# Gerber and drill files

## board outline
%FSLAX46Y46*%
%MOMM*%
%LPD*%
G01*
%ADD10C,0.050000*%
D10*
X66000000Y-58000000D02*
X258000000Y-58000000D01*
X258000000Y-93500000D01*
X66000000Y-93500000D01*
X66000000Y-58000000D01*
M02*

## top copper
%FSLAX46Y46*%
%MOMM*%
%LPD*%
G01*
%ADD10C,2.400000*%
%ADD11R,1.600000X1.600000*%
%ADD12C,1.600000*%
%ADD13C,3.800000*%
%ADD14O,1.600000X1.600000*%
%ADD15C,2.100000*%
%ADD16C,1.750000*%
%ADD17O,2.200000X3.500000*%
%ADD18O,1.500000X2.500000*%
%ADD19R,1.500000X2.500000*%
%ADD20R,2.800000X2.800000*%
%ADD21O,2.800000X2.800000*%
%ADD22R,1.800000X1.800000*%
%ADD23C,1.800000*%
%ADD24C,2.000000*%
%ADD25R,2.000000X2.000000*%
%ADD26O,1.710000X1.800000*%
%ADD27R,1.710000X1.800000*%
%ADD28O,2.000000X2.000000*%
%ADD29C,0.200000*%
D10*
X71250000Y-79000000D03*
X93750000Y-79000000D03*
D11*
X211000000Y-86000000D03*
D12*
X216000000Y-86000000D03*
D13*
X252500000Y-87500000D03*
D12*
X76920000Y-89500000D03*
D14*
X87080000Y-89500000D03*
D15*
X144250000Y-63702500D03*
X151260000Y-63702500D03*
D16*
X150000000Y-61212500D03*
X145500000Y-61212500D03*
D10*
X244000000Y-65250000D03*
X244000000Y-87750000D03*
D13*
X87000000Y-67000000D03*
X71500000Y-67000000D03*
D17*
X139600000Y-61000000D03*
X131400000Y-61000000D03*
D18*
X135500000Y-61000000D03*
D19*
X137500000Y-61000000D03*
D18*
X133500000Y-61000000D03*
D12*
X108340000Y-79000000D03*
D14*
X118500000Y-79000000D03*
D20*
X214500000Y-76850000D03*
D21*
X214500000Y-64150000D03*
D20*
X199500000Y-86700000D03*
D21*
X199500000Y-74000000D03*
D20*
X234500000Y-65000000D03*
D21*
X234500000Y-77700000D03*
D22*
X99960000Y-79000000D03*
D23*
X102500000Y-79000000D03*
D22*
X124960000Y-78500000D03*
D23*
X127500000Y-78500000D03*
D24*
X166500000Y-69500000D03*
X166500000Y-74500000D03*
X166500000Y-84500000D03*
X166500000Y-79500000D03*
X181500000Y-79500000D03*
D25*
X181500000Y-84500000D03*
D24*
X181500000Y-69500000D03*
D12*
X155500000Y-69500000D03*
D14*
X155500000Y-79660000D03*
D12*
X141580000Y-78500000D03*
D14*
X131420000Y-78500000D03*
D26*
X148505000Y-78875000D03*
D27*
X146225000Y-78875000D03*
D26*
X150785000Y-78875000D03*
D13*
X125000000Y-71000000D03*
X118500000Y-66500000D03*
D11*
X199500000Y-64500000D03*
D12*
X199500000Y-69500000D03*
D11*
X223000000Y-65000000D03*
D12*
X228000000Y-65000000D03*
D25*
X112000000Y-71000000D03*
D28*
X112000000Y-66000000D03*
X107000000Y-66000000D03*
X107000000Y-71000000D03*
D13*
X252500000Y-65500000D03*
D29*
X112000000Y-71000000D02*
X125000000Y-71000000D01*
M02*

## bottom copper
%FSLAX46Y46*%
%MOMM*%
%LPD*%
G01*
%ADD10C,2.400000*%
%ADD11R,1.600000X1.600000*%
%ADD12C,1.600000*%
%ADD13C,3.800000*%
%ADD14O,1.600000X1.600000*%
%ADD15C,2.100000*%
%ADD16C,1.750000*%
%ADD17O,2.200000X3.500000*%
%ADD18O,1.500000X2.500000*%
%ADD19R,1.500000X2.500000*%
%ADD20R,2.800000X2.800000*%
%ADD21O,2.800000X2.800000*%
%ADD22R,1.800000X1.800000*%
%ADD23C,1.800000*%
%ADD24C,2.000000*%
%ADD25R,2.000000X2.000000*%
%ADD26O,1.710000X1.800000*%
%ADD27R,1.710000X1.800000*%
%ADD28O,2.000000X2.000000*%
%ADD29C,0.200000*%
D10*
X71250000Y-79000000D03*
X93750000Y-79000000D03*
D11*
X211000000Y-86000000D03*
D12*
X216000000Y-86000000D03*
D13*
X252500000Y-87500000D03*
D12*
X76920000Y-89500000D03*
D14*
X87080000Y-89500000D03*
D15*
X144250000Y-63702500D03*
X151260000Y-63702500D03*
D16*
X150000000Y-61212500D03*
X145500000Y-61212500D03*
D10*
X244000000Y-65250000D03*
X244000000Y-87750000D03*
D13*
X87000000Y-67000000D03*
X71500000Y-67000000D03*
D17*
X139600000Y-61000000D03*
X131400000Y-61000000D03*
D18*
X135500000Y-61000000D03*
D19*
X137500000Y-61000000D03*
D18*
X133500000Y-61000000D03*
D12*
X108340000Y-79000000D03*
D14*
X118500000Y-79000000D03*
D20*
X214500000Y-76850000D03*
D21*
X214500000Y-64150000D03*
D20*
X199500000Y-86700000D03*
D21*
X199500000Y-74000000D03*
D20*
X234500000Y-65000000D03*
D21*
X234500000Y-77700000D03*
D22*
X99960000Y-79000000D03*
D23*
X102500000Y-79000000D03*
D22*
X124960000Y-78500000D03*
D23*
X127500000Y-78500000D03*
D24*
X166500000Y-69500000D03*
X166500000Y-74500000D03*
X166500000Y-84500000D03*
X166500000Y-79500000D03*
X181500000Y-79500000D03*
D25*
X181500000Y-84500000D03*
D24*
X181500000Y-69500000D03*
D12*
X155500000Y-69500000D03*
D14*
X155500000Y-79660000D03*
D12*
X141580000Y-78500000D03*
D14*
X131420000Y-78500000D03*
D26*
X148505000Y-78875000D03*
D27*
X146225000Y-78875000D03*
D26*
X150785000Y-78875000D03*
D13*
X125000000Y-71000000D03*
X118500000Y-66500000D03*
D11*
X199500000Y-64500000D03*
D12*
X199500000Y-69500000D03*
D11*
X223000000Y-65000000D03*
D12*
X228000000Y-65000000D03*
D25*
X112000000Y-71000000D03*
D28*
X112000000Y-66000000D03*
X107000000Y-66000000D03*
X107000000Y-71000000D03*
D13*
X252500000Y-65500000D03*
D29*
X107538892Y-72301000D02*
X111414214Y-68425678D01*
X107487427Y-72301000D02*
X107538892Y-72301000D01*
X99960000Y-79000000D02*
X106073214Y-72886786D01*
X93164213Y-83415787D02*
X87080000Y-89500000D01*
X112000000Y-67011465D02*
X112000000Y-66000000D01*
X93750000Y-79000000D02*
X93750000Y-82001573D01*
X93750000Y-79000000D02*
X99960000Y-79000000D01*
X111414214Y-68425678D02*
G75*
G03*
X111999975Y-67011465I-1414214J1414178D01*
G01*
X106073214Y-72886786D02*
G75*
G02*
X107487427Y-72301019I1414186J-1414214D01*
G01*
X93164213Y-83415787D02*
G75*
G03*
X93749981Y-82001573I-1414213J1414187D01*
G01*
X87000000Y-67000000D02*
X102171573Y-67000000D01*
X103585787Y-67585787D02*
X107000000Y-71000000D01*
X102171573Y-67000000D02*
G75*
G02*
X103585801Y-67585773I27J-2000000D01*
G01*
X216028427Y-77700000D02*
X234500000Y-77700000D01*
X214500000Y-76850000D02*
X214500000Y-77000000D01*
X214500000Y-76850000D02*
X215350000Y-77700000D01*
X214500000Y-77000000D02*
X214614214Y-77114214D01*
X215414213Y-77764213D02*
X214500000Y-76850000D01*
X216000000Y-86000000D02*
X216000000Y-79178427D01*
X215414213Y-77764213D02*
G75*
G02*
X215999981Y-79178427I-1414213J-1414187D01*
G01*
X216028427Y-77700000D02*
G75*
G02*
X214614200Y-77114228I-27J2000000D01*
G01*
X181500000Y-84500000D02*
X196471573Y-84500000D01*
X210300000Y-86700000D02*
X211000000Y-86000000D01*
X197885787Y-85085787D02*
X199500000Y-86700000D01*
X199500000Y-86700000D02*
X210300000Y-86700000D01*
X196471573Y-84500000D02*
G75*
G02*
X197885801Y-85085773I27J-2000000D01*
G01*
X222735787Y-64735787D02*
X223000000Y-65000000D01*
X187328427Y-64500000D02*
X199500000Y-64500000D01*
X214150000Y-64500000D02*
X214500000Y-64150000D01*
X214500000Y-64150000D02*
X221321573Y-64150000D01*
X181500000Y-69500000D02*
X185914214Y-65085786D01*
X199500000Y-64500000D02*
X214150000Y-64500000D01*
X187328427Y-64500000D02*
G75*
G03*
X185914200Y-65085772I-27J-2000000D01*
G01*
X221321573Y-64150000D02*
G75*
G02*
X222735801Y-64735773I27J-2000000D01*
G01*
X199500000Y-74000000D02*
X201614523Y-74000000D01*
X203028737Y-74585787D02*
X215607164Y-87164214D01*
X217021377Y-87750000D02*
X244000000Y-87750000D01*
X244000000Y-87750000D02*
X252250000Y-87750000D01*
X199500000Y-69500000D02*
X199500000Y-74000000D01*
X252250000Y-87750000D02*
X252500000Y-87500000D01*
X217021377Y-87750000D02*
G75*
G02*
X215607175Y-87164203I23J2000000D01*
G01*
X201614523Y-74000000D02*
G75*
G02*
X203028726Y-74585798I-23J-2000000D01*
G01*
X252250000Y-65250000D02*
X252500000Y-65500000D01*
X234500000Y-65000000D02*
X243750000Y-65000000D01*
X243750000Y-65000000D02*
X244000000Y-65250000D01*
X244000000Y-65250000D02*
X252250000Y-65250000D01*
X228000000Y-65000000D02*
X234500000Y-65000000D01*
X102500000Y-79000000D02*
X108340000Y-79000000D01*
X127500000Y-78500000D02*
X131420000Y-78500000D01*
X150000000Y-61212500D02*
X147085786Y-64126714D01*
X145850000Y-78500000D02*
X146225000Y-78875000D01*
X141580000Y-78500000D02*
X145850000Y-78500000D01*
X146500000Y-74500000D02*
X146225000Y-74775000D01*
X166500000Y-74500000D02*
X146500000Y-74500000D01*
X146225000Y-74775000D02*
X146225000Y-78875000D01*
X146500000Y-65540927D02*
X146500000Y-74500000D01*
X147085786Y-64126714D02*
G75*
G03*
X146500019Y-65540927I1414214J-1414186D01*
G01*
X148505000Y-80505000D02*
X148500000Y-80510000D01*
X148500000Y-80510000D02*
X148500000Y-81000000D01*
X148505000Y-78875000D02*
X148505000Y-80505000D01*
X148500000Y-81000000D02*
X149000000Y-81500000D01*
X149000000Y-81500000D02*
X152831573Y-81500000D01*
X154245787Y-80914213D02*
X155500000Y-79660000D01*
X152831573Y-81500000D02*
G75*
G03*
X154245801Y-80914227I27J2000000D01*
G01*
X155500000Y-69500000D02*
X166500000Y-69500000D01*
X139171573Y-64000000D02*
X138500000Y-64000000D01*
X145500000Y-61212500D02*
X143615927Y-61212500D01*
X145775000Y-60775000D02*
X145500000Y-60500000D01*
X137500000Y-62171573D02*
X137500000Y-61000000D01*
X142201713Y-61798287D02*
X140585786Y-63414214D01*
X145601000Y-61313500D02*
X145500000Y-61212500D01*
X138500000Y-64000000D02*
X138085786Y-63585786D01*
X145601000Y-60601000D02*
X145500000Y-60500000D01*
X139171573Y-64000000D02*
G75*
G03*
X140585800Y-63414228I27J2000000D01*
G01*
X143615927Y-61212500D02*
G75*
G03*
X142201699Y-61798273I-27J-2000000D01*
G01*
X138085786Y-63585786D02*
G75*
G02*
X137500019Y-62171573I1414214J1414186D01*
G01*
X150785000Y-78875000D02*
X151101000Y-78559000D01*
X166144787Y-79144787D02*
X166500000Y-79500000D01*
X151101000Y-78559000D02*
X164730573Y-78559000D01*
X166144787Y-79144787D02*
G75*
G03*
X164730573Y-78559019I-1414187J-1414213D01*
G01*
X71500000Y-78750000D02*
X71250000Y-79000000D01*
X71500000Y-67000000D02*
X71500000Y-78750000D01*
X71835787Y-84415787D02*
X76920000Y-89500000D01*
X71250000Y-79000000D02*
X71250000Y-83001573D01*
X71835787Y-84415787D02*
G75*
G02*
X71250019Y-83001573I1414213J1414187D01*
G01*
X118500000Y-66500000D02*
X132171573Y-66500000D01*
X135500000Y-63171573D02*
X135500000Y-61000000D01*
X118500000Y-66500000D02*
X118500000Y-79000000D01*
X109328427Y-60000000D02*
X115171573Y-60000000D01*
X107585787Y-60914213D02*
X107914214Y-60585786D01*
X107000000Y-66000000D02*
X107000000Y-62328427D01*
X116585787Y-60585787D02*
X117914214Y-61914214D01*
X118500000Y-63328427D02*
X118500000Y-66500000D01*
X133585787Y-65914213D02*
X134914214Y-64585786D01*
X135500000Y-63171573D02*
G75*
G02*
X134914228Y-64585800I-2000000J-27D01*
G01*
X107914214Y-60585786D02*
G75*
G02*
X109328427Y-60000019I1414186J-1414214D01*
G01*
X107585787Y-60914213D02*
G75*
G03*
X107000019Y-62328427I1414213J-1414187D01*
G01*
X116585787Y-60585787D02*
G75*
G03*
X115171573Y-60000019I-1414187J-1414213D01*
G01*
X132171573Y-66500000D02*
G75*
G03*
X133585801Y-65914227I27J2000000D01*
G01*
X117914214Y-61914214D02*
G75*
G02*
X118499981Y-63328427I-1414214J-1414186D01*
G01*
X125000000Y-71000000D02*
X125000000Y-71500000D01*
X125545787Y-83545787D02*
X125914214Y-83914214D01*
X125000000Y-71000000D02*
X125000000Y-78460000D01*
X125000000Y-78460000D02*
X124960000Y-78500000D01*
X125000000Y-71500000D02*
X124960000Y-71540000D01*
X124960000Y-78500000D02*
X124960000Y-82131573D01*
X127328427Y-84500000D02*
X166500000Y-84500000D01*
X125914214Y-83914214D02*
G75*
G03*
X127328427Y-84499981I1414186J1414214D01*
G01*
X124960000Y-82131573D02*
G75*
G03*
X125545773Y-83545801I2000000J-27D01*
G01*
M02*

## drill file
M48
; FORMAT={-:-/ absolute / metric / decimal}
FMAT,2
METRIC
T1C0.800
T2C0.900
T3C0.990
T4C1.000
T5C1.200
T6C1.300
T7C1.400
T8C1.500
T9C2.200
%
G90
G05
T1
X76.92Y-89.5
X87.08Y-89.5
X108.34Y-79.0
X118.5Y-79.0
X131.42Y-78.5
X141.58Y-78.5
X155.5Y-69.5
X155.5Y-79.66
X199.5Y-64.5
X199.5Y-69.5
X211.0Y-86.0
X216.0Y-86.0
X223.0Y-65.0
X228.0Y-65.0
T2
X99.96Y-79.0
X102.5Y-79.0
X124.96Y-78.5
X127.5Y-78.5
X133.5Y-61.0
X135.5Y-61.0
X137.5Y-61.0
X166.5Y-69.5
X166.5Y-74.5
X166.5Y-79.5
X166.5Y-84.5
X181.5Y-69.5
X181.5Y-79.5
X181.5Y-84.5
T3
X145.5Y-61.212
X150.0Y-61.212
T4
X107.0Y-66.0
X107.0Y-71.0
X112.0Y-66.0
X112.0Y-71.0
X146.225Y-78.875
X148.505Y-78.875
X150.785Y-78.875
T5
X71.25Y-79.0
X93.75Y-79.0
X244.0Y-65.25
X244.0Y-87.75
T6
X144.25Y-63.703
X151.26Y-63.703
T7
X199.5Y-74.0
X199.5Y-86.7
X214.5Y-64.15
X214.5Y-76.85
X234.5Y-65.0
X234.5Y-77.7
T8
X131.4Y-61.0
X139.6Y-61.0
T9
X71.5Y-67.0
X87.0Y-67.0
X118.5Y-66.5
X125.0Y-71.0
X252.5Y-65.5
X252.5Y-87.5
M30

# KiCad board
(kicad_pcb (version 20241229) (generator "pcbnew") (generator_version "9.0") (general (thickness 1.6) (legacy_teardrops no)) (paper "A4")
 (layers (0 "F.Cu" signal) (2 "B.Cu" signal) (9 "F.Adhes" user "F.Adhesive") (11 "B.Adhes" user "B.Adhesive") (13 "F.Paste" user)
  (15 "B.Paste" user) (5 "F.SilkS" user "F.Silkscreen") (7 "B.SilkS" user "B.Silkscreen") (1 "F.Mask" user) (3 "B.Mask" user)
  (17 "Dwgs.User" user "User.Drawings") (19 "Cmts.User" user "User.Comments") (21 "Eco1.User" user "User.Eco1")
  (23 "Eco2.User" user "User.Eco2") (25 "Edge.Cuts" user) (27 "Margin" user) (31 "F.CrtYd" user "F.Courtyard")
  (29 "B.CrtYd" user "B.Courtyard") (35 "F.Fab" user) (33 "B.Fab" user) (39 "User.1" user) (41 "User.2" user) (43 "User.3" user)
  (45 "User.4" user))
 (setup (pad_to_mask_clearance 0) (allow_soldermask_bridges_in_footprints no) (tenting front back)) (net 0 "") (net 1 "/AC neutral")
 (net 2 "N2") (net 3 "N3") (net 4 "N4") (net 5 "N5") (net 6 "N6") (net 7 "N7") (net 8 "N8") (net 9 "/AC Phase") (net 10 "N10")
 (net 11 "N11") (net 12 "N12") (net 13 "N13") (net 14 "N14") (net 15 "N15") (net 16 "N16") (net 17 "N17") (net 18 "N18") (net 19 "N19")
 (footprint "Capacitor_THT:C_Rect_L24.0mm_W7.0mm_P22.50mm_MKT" (layer "F.Cu") (at 71.25 79)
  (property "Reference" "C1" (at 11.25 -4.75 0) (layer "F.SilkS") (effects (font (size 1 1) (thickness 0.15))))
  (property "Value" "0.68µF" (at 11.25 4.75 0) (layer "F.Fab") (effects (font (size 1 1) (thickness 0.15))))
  (pad "1" thru_hole circle (at 0 0) (size 2.4 2.4) (drill 1.2) (layers "*.Cu" "*.Mask") (remove_unused_layers no) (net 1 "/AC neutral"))
  (pad "2" thru_hole circle (at 22.5 0) (size 2.4 2.4) (drill 1.2) (layers "*.Cu" "*.Mask") (remove_unused_layers no) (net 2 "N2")))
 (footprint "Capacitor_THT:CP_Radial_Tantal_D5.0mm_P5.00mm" (layer "F.Cu") (at 211 86)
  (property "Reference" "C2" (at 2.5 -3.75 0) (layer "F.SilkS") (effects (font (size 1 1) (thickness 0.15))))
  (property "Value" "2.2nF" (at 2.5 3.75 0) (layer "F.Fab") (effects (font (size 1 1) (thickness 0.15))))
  (pad "1" thru_hole rect (at 0 0) (size 1.6 1.6) (drill 0.8) (layers "*.Cu" "*.Mask") (remove_unused_layers no) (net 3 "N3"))
  (pad "2" thru_hole circle (at 5 0) (size 1.6 1.6) (drill 0.8) (layers "*.Cu" "*.Mask") (remove_unused_layers no) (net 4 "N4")))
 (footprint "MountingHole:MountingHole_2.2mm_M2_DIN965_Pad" (layer "F.Cu") (at 252.5 87.5)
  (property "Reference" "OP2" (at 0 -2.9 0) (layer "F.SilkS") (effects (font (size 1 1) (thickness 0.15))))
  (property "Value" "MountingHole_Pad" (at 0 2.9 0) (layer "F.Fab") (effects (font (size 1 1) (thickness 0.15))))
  (pad "1" thru_hole circle (at 0 0) (size 3.8 3.8) (drill 2.2) (layers "*.Cu" "*.Mask") (remove_unused_layers no) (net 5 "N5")))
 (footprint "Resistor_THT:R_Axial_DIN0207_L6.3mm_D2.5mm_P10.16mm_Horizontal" (layer "F.Cu") (at 76.92 89.5)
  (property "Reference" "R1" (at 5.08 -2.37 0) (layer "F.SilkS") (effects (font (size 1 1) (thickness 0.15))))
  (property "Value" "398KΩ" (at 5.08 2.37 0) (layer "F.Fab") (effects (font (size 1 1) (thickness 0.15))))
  (pad "1" thru_hole circle (at 0 0) (size 1.6 1.6) (drill 0.8) (layers "*.Cu" "*.Mask") (remove_unused_layers no) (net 1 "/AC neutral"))
  (pad "2" thru_hole oval (at 10.16 0) (size 1.6 1.6) (drill 0.8) (layers "*.Cu" "*.Mask") (remove_unused_layers no) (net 2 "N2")))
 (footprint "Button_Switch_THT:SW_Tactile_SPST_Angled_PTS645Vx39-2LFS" (layer "F.Cu") (at 145.5 61.2125)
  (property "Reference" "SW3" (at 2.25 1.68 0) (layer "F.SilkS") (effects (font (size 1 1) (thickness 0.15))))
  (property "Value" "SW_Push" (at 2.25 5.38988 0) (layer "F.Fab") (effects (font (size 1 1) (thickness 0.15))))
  (pad "" thru_hole circle (at -1.25 2.49) (size 2.1 2.1) (drill 1.3) (layers "*.Cu" "*.Mask") (remove_unused_layers no))
  (pad "" thru_hole circle (at 5.76 2.49) (size 2.1 2.1) (drill 1.3) (layers "*.Cu" "*.Mask") (remove_unused_layers no))
  (pad "1" thru_hole circle (at 4.5 0) (size 1.75 1.75) (drill 0.99) (layers "*.Cu" "*.Mask") (remove_unused_layers no) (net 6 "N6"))
  (pad "2" thru_hole circle (at 0 0) (size 1.75 1.75) (drill 0.99) (layers "*.Cu" "*.Mask") (remove_unused_layers no) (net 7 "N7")))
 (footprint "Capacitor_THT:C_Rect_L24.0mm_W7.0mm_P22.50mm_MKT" (layer "F.Cu") (at 244 65.25 -90)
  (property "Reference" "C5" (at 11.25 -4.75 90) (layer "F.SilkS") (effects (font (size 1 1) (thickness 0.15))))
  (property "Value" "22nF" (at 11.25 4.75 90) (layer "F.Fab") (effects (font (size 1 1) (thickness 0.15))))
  (pad "1" thru_hole circle (at 0 0 270) (size 2.4 2.4) (drill 1.2) (layers "*.Cu" "*.Mask") (remove_unused_layers no) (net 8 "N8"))
  (pad "2" thru_hole circle (at 22.5 0 270) (size 2.4 2.4) (drill 1.2) (layers "*.Cu" "*.Mask") (remove_unused_layers no) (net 5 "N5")))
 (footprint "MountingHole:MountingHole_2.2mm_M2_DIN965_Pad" (layer "F.Cu") (at 87 67)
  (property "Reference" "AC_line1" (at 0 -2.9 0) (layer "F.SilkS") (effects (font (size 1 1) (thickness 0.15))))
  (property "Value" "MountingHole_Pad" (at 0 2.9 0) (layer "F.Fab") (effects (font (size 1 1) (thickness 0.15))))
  (pad "1" thru_hole circle (at 0 0) (size 3.8 3.8) (drill 2.2) (layers "*.Cu" "*.Mask") (remove_unused_layers no) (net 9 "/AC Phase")))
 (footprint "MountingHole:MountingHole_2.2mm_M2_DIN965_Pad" (layer "F.Cu") (at 71.5 67)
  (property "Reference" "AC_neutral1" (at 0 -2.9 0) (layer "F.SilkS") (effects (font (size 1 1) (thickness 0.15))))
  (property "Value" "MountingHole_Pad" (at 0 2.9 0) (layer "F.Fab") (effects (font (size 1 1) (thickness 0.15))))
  (pad "1" thru_hole circle (at 0 0) (size 3.8 3.8) (drill 2.2) (layers "*.Cu" "*.Mask") (remove_unused_layers no) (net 1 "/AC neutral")))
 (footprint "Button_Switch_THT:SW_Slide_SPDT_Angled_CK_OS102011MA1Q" (layer "F.Cu") (at 137.5 61 180)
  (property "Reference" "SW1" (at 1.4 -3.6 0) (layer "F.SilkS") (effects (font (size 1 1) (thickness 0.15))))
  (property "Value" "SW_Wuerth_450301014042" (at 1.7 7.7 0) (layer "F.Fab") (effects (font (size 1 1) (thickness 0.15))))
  (pad "" thru_hole oval (at -2.1 0 180) (size 2.2 3.5) (drill 1.5) (layers "*.Cu" "*.Mask") (remove_unused_layers no))
  (pad "" thru_hole oval (at 6.1 0 180) (size 2.2 3.5) (drill 1.5) (layers "*.Cu" "*.Mask") (remove_unused_layers no))
  (pad "1" thru_hole oval (at 2 0 180) (size 1.5 2.5) (drill 0.9) (layers "*.Cu" "*.Mask") (remove_unused_layers no) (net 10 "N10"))
  (pad "2" thru_hole rect (at 0 0 180) (size 1.5 2.5) (drill 0.9) (layers "*.Cu" "*.Mask") (remove_unused_layers no) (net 7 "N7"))
  (pad "3" thru_hole oval (at 4 0 180) (size 1.5 2.5) (drill 0.9) (layers "*.Cu" "*.Mask") (remove_unused_layers no) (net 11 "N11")))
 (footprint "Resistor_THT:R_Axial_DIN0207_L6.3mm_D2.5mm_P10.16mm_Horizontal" (layer "F.Cu") (at 108.34 79)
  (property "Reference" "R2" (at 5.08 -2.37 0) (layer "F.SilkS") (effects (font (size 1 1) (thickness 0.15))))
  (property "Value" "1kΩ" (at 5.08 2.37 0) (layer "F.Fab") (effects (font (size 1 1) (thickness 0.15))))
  (pad "1" thru_hole circle (at 0 0) (size 1.6 1.6) (drill 0.8) (layers "*.Cu" "*.Mask") (remove_unused_layers no) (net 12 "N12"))
  (pad "2" thru_hole oval (at 10.16 0) (size 1.6 1.6) (drill 0.8) (layers "*.Cu" "*.Mask") (remove_unused_layers no) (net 10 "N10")))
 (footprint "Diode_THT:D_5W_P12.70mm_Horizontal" (layer "F.Cu") (at 214.5 76.85 90)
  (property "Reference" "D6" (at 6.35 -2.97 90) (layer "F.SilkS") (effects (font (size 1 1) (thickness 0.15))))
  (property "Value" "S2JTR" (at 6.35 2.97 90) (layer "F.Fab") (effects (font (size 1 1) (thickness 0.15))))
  (pad "1" thru_hole rect (at 0 0 90) (size 2.8 2.8) (drill 1.4) (layers "*.Cu" "*.Mask") (remove_unused_layers no) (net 4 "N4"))
  (pad "2" thru_hole oval (at 12.7 0 90) (size 2.8 2.8) (drill 1.4) (layers "*.Cu" "*.Mask") (remove_unused_layers no) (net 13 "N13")))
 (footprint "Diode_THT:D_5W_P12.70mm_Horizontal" (layer "F.Cu") (at 199.5 86.7 90)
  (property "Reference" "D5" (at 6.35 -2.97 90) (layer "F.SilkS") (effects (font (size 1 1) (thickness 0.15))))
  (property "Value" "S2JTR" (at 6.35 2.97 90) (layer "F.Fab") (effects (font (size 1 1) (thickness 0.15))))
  (pad "1" thru_hole rect (at 0 0 90) (size 2.8 2.8) (drill 1.4) (layers "*.Cu" "*.Mask") (remove_unused_layers no) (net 3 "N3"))
  (pad "2" thru_hole oval (at 12.7 0 90) (size 2.8 2.8) (drill 1.4) (layers "*.Cu" "*.Mask") (remove_unused_layers no) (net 5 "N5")))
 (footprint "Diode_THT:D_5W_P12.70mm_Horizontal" (layer "F.Cu") (at 234.5 65 -90)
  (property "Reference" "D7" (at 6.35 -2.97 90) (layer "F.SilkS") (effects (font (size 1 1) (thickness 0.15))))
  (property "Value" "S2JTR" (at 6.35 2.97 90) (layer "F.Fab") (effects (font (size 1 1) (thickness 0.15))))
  (pad "1" thru_hole rect (at 0 0 270) (size 2.8 2.8) (drill 1.4) (layers "*.Cu" "*.Mask") (remove_unused_layers no) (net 8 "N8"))
  (pad "2" thru_hole oval (at 12.7 0 270) (size 2.8 2.8) (drill 1.4) (layers "*.Cu" "*.Mask") (remove_unused_layers no) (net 4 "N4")))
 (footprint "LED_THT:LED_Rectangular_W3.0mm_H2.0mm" (layer "F.Cu") (at 99.96 79)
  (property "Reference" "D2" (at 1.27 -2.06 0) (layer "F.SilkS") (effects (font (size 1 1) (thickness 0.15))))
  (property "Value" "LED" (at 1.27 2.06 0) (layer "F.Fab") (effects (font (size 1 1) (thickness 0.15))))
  (pad "1" thru_hole rect (at 0 0) (size 1.8 1.8) (drill 0.9) (layers "*.Cu" "*.Mask") (remove_unused_layers no) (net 2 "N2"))
  (pad "2" thru_hole circle (at 2.54 0) (size 1.8 1.8) (drill 0.9) (layers "*.Cu" "*.Mask") (remove_unused_layers no) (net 12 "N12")))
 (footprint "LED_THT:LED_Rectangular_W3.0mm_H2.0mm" (layer "F.Cu") (at 124.96 78.5)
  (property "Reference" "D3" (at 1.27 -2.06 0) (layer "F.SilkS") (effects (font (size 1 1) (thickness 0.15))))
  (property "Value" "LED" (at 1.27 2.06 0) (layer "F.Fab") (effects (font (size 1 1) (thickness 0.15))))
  (pad "1" thru_hole rect (at 0 0) (size 1.8 1.8) (drill 0.9) (layers "*.Cu" "*.Mask") (remove_unused_layers no) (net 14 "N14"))
  (pad "2" thru_hole circle (at 2.54 0) (size 1.8 1.8) (drill 0.9) (layers "*.Cu" "*.Mask") (remove_unused_layers no) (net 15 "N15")))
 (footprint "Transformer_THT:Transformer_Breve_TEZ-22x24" (layer "F.Cu") (at 181.5 84.5 90)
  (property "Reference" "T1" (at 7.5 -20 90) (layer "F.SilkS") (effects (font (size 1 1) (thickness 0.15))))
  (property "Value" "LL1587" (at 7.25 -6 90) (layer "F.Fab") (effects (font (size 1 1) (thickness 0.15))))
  (pad "1" thru_hole circle (at 15 -15 90) (size 2 2) (drill 0.9) (layers "*.Cu" "*.Mask") (remove_unused_layers no) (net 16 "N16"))
  (pad "2" thru_hole circle (at 10 -15 90) (size 2 2) (drill 0.9) (layers "*.Cu" "*.Mask") (remove_unused_layers no) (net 6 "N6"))
  (pad "3" thru_hole circle (at 0 -15 90) (size 2 2) (drill 0.9) (layers "*.Cu" "*.Mask") (remove_unused_layers no) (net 14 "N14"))
  (pad "4" thru_hole circle (at 5 -15 90) (size 2 2) (drill 0.9) (layers "*.Cu" "*.Mask") (remove_unused_layers no) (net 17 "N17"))
  (pad "5" thru_hole circle (at 5 0 90) (size 2 2) (drill 0.9) (layers "*.Cu" "*.Mask") (remove_unused_layers no) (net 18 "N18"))
  (pad "6" thru_hole rect (at 0 0 90) (size 2 2) (drill 0.9) (layers "*.Cu" "*.Mask") (remove_unused_layers no) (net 3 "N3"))
  (pad "8" thru_hole circle (at 15 0 90) (size 2 2) (drill 0.9) (layers "*.Cu" "*.Mask") (remove_unused_layers no) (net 13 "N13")))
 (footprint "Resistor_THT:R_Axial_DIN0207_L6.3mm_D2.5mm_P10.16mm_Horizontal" (layer "F.Cu") (at 155.5 69.5 -90)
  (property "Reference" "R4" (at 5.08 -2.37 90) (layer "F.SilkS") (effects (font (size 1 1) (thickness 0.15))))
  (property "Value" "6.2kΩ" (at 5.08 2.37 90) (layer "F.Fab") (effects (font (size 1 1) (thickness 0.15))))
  (pad "1" thru_hole circle (at 0 0 270) (size 1.6 1.6) (drill 0.8) (layers "*.Cu" "*.Mask") (remove_unused_layers no) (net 16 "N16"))
  (pad "2" thru_hole oval (at 10.16 0 270) (size 1.6 1.6) (drill 0.8) (layers "*.Cu" "*.Mask") (remove_unused_layers no) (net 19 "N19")))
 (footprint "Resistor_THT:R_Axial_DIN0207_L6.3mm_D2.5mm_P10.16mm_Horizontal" (layer "F.Cu") (at 141.58 78.5 180)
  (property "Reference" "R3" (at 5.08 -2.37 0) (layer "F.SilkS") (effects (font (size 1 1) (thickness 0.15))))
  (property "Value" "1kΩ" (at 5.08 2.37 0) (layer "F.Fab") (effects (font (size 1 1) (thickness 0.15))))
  (pad "1" thru_hole circle (at 0 0 180) (size 1.6 1.6) (drill 0.8) (layers "*.Cu" "*.Mask") (remove_unused_layers no) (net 6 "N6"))
  (pad "2" thru_hole oval (at 10.16 0 180) (size 1.6 1.6) (drill 0.8) (layers "*.Cu" "*.Mask") (remove_unused_layers no) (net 15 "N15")))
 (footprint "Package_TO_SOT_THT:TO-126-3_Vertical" (layer "F.Cu") (at 146.225 78.875)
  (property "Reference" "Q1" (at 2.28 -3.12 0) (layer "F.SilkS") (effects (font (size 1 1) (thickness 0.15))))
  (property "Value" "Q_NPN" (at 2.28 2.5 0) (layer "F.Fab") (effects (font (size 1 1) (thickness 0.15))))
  (pad "B" thru_hole oval (at 2.28 0) (size 1.71 1.8) (drill 1) (layers "*.Cu" "*.Mask") (remove_unused_layers no) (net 19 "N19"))
  (pad "C" thru_hole rect (at 0 0) (size 1.71 1.8) (drill 1) (layers "*.Cu" "*.Mask") (remove_unused_layers no) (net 6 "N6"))
  (pad "E" thru_hole oval (at 4.56 0) (size 1.71 1.8) (drill 1) (layers "*.Cu" "*.Mask") (remove_unused_layers no) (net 17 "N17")))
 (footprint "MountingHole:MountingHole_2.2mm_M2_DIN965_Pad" (layer "F.Cu") (at 125 71)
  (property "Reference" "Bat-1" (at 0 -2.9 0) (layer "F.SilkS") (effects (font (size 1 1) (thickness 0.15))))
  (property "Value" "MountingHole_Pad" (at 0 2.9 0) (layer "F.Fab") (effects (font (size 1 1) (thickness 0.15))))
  (pad "1" thru_hole circle (at 0 0) (size 3.8 3.8) (drill 2.2) (layers "*.Cu" "*.Mask") (remove_unused_layers no) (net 14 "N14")))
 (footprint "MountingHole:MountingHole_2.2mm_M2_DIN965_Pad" (layer "F.Cu") (at 118.5 66.5)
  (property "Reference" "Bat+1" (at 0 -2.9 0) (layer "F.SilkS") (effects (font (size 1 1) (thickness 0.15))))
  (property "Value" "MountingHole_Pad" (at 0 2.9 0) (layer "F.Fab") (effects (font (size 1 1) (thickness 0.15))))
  (pad "1" thru_hole circle (at 0 0) (size 3.8 3.8) (drill 2.2) (layers "*.Cu" "*.Mask") (remove_unused_layers no) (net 10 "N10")))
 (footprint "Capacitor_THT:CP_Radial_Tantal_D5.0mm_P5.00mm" (layer "F.Cu") (at 199.5 64.5 -90)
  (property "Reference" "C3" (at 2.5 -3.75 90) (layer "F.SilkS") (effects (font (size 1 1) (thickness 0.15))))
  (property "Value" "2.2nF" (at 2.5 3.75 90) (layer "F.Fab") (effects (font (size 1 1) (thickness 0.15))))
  (pad "1" thru_hole rect (at 0 0 270) (size 1.6 1.6) (drill 0.8) (layers "*.Cu" "*.Mask") (remove_unused_layers no) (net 13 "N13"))
  (pad "2" thru_hole circle (at 5 0 270) (size 1.6 1.6) (drill 0.8) (layers "*.Cu" "*.Mask") (remove_unused_layers no) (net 5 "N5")))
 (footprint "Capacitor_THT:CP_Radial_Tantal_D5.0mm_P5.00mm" (layer "F.Cu") (at 223 65)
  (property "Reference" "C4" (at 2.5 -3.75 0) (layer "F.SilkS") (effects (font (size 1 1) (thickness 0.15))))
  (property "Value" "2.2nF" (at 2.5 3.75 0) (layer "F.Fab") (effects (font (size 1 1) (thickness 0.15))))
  (pad "1" thru_hole rect (at 0 0) (size 1.6 1.6) (drill 0.8) (layers "*.Cu" "*.Mask") (remove_unused_layers no) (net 13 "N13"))
  (pad "2" thru_hole circle (at 5 0) (size 1.6 1.6) (drill 0.8) (layers "*.Cu" "*.Mask") (remove_unused_layers no) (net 8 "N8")))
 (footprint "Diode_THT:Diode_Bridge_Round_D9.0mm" (layer "F.Cu") (at 112 71 180)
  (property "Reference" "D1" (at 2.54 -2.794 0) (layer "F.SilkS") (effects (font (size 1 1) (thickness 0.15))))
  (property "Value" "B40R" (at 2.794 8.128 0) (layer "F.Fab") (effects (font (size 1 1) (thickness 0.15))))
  (pad "1" thru_hole rect (at 0 0 180) (size 2 2) (drill 1) (layers "*.Cu" "*.Mask") (remove_unused_layers no) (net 14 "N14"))
  (pad "2" thru_hole oval (at 0 5 180) (size 2 2) (drill 1) (layers "*.Cu" "*.Mask") (remove_unused_layers no) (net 2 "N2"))
  (pad "3" thru_hole oval (at 5 5 180) (size 2 2) (drill 1) (layers "*.Cu" "*.Mask") (remove_unused_layers no) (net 10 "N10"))
  (pad "4" thru_hole oval (at 5 0 180) (size 2 2) (drill 1) (layers "*.Cu" "*.Mask") (remove_unused_layers no) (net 9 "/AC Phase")))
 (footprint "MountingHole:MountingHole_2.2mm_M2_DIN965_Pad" (layer "F.Cu") (at 252.5 65.5)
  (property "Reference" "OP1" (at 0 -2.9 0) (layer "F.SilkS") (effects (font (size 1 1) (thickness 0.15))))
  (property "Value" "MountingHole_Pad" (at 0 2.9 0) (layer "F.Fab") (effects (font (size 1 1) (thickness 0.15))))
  (pad "1" thru_hole circle (at 0 0) (size 3.8 3.8) (drill 2.2) (layers "*.Cu" "*.Mask") (remove_unused_layers no) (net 8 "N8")))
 (gr_rect (start 66 58) (end 258 93.5) (stroke (width 0.05) (type default)) (fill no) (layer "Edge.Cuts"))
 (segment (start 107.538892 72.301) (end 111.414214 68.425678) (width 0.2) (layer "B.Cu") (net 2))
 (segment (start 107.487427 72.301) (end 107.538892 72.301) (width 0.2) (layer "B.Cu") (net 2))
 (segment (start 99.96 79) (end 106.073214 72.886786) (width 0.2) (layer "B.Cu") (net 2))
 (segment (start 93.164213 83.415787) (end 87.08 89.5) (width 0.2) (layer "B.Cu") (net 2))
 (segment (start 112 67.011465) (end 112 66) (width 0.2) (layer "B.Cu") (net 2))
 (segment (start 93.75 79) (end 93.75 82.001573) (width 0.2) (layer "B.Cu") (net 2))
 (segment (start 93.75 79) (end 99.96 79) (width 0.2) (layer "B.Cu") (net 2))
 (arc (start 111.414214 68.425678) (mid 111.847759 67.776832) (end 112 67.011465) (width 0.2) (layer "B.Cu") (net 2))
 (arc (start 106.073214 72.886786) (mid 106.72206 72.453241) (end 107.487427 72.301) (width 0.2) (layer "B.Cu") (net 2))
 (arc (start 93.164213 83.415787) (mid 93.597759 82.76694) (end 93.75 82.001573) (width 0.2) (layer "B.Cu") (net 2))
 (segment (start 87 67) (end 102.171573 67) (width 0.2) (layer "B.Cu") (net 9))
 (segment (start 103.585787 67.585787) (end 107 71) (width 0.2) (layer "B.Cu") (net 9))
 (arc (start 102.171573 67) (mid 102.93694 67.152241) (end 103.585787 67.585787) (width 0.2) (layer "B.Cu") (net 9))
 (segment (start 216.028427 77.7) (end 234.5 77.7) (width 0.2) (layer "B.Cu") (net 4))
 (segment (start 214.5 76.85) (end 214.5 77) (width 0.2) (layer "B.Cu") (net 4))
 (segment (start 214.5 76.85) (end 215.35 77.7) (width 0.2) (layer "B.Cu") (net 4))
 (segment (start 214.5 77) (end 214.614214 77.114214) (width 0.2) (layer "B.Cu") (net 4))
 (segment (start 215.414213 77.764213) (end 214.5 76.85) (width 0.2) (layer "B.Cu") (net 4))
 (segment (start 216 86) (end 216 79.178427) (width 0.2) (layer "B.Cu") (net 4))
 (arc (start 215.414213 77.764213) (mid 215.847759 78.41306) (end 216 79.178427) (width 0.2) (layer "B.Cu") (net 4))
 (arc (start 216.028427 77.7) (mid 215.26306 77.547759) (end 214.614214 77.114214) (width 0.2) (layer "B.Cu") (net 4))
 (segment (start 181.5 84.5) (end 196.471573 84.5) (width 0.2) (layer "B.Cu") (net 3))
 (segment (start 210.3 86.7) (end 211 86) (width 0.2) (layer "B.Cu") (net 3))
 (segment (start 197.885787 85.085787) (end 199.5 86.7) (width 0.2) (layer "B.Cu") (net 3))
 (segment (start 199.5 86.7) (end 210.3 86.7) (width 0.2) (layer "B.Cu") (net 3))
 (arc (start 196.471573 84.5) (mid 197.23694 84.652241) (end 197.885787 85.085787) (width 0.2) (layer "B.Cu") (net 3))
 (segment (start 222.735787 64.735787) (end 223 65) (width 0.2) (layer "B.Cu") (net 13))
 (segment (start 187.328427 64.5) (end 199.5 64.5) (width 0.2) (layer "B.Cu") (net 13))
 (segment (start 214.15 64.5) (end 214.5 64.15) (width 0.2) (layer "B.Cu") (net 13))
 (segment (start 214.5 64.15) (end 221.321573 64.15) (width 0.2) (layer "B.Cu") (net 13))
 (segment (start 181.5 69.5) (end 185.914214 65.085786) (width 0.2) (layer "B.Cu") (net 13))
 (segment (start 199.5 64.5) (end 214.15 64.5) (width 0.2) (layer "B.Cu") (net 13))
 (arc (start 187.328427 64.5) (mid 186.56306 64.652241) (end 185.914214 65.085786) (width 0.2) (layer "B.Cu") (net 13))
 (arc (start 221.321573 64.15) (mid 222.08694 64.302241) (end 222.735787 64.735787) (width 0.2) (layer "B.Cu") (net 13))
 (segment (start 199.5 74) (end 201.614523 74) (width 0.2) (layer "B.Cu") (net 5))
 (segment (start 203.028737 74.585787) (end 215.607164 87.164214) (width 0.2) (layer "B.Cu") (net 5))
 (segment (start 217.021377 87.75) (end 244 87.75) (width 0.2) (layer "B.Cu") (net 5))
 (segment (start 244 87.75) (end 252.25 87.75) (width 0.2) (layer "B.Cu") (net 5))
 (segment (start 199.5 69.5) (end 199.5 74) (width 0.2) (layer "B.Cu") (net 5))
 (segment (start 252.25 87.75) (end 252.5 87.5) (width 0.2) (layer "B.Cu") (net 5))
 (arc (start 217.021377 87.75) (mid 216.25601 87.597759) (end 215.607164 87.164214) (width 0.2) (layer "B.Cu") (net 5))
 (arc (start 201.614523 74) (mid 202.37989 74.152241) (end 203.028737 74.585787) (width 0.2) (layer "B.Cu") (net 5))
 (segment (start 252.25 65.25) (end 252.5 65.5) (width 0.2) (layer "B.Cu") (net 8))
 (segment (start 234.5 65) (end 243.75 65) (width 0.2) (layer "B.Cu") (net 8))
 (segment (start 243.75 65) (end 244 65.25) (width 0.2) (layer "B.Cu") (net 8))
 (segment (start 244 65.25) (end 252.25 65.25) (width 0.2) (layer "B.Cu") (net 8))
 (segment (start 228 65) (end 234.5 65) (width 0.2) (layer "B.Cu") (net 8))
 (segment (start 102.5 79) (end 108.34 79) (width 0.2) (layer "B.Cu") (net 12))
 (segment (start 127.5 78.5) (end 131.42 78.5) (width 0.2) (layer "B.Cu") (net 15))
 (segment (start 150 61.2125) (end 147.085786 64.126714) (width 0.2) (layer "B.Cu") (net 6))
 (segment (start 145.85 78.5) (end 146.225 78.875) (width 0.2) (layer "B.Cu") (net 6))
 (segment (start 141.58 78.5) (end 145.85 78.5) (width 0.2) (layer "B.Cu") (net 6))
 (segment (start 146.5 74.5) (end 146.225 74.775) (width 0.2) (layer "B.Cu") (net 6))
 (segment (start 166.5 74.5) (end 146.5 74.5) (width 0.2) (layer "B.Cu") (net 6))
 (segment (start 146.225 74.775) (end 146.225 78.875) (width 0.2) (layer "B.Cu") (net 6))
 (segment (start 146.5 65.540927) (end 146.5 74.5) (width 0.2) (layer "B.Cu") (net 6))
 (arc (start 147.085786 64.126714) (mid 146.652241 64.77556) (end 146.5 65.540927) (width 0.2) (layer "B.Cu") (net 6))
 (segment (start 148.505 80.505) (end 148.5 80.51) (width 0.2) (layer "B.Cu") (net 19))
 (segment (start 148.5 80.51) (end 148.5 81) (width 0.2) (layer "B.Cu") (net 19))
 (segment (start 148.505 78.875) (end 148.505 80.505) (width 0.2) (layer "B.Cu") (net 19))
 (segment (start 148.5 81) (end 149 81.5) (width 0.2) (layer "B.Cu") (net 19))
 (segment (start 149 81.5) (end 152.831573 81.5) (width 0.2) (layer "B.Cu") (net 19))
 (segment (start 154.245787 80.914213) (end 155.5 79.66) (width 0.2) (layer "B.Cu") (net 19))
 (arc (start 152.831573 81.5) (mid 153.59694 81.347759) (end 154.245787 80.914213) (width 0.2) (layer "B.Cu") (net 19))
 (segment (start 155.5 69.5) (end 166.5 69.5) (width 0.2) (layer "B.Cu") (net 16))
 (segment (start 139.171573 64) (end 138.5 64) (width 0.2) (layer "B.Cu") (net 7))
 (segment (start 145.5 61.2125) (end 143.615927 61.2125) (width 0.2) (layer "B.Cu") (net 7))
 (segment (start 145.775 60.775) (end 145.5 60.5) (width 0.2) (layer "B.Cu") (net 7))
 (segment (start 137.5 62.171573) (end 137.5 61) (width 0.2) (layer "B.Cu") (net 7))
 (segment (start 142.201713 61.798287) (end 140.585786 63.414214) (width 0.2) (layer "B.Cu") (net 7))
 (segment (start 145.601 61.3135) (end 145.5 61.2125) (width 0.2) (layer "B.Cu") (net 7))
 (segment (start 138.5 64) (end 138.085786 63.585786) (width 0.2) (layer "B.Cu") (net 7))
 (segment (start 145.601 60.601) (end 145.5 60.5) (width 0.2) (layer "B.Cu") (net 7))
 (arc (start 139.171573 64) (mid 139.93694 63.847759) (end 140.585786 63.414214) (width 0.2) (layer "B.Cu") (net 7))
 (arc (start 143.615927 61.2125) (mid 142.85056 61.364741) (end 142.201713 61.798287) (width 0.2) (layer "B.Cu") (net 7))
 (arc (start 138.085786 63.585786) (mid 137.652241 62.93694) (end 137.5 62.171573) (width 0.2) (layer "B.Cu") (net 7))
 (segment (start 150.785 78.875) (end 151.101 78.559) (width 0.2) (layer "B.Cu") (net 17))
 (segment (start 166.144787 79.144787) (end 166.5 79.5) (width 0.2) (layer "B.Cu") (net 17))
 (segment (start 151.101 78.559) (end 164.730573 78.559) (width 0.2) (layer "B.Cu") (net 17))
 (arc (start 166.144787 79.144787) (mid 165.49594 78.711241) (end 164.730573 78.559) (width 0.2) (layer "B.Cu") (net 17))
 (segment (start 71.5 78.75) (end 71.25 79) (width 0.2) (layer "B.Cu") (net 1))
 (segment (start 71.5 67) (end 71.5 78.75) (width 0.2) (layer "B.Cu") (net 1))
 (segment (start 71.835787 84.415787) (end 76.92 89.5) (width 0.2) (layer "B.Cu") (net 1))
 (segment (start 71.25 79) (end 71.25 83.001573) (width 0.2) (layer "B.Cu") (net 1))
 (arc (start 71.835787 84.415787) (mid 71.402241 83.76694) (end 71.25 83.001573) (width 0.2) (layer "B.Cu") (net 1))
 (segment (start 118.5 66.5) (end 132.171573 66.5) (width 0.2) (layer "B.Cu") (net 10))
 (segment (start 135.5 63.171573) (end 135.5 61) (width 0.2) (layer "B.Cu") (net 10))
 (segment (start 118.5 66.5) (end 118.5 79) (width 0.2) (layer "B.Cu") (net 10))
 (segment (start 109.328427 60) (end 115.171573 60) (width 0.2) (layer "B.Cu") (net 10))
 (segment (start 107.585787 60.914213) (end 107.914214 60.585786) (width 0.2) (layer "B.Cu") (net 10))
 (segment (start 107 66) (end 107 62.328427) (width 0.2) (layer "B.Cu") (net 10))
 (segment (start 116.585787 60.585787) (end 117.914214 61.914214) (width 0.2) (layer "B.Cu") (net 10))
 (segment (start 118.5 63.328427) (end 118.5 66.5) (width 0.2) (layer "B.Cu") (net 10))
 (segment (start 133.585787 65.914213) (end 134.914214 64.585786) (width 0.2) (layer "B.Cu") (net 10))
 (arc (start 135.5 63.171573) (mid 135.347759 63.93694) (end 134.914214 64.585786) (width 0.2) (layer "B.Cu") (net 10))
 (arc (start 107.914214 60.585786) (mid 108.56306 60.152241) (end 109.328427 60) (width 0.2) (layer "B.Cu") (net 10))
 (arc (start 107.585787 60.914213) (mid 107.152241 61.56306) (end 107 62.328427) (width 0.2) (layer "B.Cu") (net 10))
 (arc (start 116.585787 60.585787) (mid 115.93694 60.152241) (end 115.171573 60) (width 0.2) (layer "B.Cu") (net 10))
 (arc (start 132.171573 66.5) (mid 132.93694 66.347759) (end 133.585787 65.914213) (width 0.2) (layer "B.Cu") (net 10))
 (arc (start 117.914214 61.914214) (mid 118.347759 62.56306) (end 118.5 63.328427) (width 0.2) (layer "B.Cu") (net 10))
 (segment (start 112 71) (end 125 71) (width 0.2) (layer "F.Cu") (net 14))
 (segment (start 125 71) (end 125 71.5) (width 0.2) (layer "B.Cu") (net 14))
 (segment (start 125.545787 83.545787) (end 125.914214 83.914214) (width 0.2) (layer "B.Cu") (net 14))
 (segment (start 125 71) (end 125 78.46) (width 0.2) (layer "B.Cu") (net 14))
 (segment (start 125 78.46) (end 124.96 78.5) (width 0.2) (layer "B.Cu") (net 14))
 (segment (start 125 71.5) (end 124.96 71.54) (width 0.2) (layer "B.Cu") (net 14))
 (segment (start 124.96 78.5) (end 124.96 82.131573) (width 0.2) (layer "B.Cu") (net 14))
 (segment (start 127.328427 84.5) (end 166.5 84.5) (width 0.2) (layer "B.Cu") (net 14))
 (arc (start 125.914214 83.914214) (mid 126.56306 84.347759) (end 127.328427 84.5) (width 0.2) (layer "B.Cu") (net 14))
 (arc (start 124.96 82.131573) (mid 125.112241 82.89694) (end 125.545787 83.545787) (width 0.2) (layer "B.Cu") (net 14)))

